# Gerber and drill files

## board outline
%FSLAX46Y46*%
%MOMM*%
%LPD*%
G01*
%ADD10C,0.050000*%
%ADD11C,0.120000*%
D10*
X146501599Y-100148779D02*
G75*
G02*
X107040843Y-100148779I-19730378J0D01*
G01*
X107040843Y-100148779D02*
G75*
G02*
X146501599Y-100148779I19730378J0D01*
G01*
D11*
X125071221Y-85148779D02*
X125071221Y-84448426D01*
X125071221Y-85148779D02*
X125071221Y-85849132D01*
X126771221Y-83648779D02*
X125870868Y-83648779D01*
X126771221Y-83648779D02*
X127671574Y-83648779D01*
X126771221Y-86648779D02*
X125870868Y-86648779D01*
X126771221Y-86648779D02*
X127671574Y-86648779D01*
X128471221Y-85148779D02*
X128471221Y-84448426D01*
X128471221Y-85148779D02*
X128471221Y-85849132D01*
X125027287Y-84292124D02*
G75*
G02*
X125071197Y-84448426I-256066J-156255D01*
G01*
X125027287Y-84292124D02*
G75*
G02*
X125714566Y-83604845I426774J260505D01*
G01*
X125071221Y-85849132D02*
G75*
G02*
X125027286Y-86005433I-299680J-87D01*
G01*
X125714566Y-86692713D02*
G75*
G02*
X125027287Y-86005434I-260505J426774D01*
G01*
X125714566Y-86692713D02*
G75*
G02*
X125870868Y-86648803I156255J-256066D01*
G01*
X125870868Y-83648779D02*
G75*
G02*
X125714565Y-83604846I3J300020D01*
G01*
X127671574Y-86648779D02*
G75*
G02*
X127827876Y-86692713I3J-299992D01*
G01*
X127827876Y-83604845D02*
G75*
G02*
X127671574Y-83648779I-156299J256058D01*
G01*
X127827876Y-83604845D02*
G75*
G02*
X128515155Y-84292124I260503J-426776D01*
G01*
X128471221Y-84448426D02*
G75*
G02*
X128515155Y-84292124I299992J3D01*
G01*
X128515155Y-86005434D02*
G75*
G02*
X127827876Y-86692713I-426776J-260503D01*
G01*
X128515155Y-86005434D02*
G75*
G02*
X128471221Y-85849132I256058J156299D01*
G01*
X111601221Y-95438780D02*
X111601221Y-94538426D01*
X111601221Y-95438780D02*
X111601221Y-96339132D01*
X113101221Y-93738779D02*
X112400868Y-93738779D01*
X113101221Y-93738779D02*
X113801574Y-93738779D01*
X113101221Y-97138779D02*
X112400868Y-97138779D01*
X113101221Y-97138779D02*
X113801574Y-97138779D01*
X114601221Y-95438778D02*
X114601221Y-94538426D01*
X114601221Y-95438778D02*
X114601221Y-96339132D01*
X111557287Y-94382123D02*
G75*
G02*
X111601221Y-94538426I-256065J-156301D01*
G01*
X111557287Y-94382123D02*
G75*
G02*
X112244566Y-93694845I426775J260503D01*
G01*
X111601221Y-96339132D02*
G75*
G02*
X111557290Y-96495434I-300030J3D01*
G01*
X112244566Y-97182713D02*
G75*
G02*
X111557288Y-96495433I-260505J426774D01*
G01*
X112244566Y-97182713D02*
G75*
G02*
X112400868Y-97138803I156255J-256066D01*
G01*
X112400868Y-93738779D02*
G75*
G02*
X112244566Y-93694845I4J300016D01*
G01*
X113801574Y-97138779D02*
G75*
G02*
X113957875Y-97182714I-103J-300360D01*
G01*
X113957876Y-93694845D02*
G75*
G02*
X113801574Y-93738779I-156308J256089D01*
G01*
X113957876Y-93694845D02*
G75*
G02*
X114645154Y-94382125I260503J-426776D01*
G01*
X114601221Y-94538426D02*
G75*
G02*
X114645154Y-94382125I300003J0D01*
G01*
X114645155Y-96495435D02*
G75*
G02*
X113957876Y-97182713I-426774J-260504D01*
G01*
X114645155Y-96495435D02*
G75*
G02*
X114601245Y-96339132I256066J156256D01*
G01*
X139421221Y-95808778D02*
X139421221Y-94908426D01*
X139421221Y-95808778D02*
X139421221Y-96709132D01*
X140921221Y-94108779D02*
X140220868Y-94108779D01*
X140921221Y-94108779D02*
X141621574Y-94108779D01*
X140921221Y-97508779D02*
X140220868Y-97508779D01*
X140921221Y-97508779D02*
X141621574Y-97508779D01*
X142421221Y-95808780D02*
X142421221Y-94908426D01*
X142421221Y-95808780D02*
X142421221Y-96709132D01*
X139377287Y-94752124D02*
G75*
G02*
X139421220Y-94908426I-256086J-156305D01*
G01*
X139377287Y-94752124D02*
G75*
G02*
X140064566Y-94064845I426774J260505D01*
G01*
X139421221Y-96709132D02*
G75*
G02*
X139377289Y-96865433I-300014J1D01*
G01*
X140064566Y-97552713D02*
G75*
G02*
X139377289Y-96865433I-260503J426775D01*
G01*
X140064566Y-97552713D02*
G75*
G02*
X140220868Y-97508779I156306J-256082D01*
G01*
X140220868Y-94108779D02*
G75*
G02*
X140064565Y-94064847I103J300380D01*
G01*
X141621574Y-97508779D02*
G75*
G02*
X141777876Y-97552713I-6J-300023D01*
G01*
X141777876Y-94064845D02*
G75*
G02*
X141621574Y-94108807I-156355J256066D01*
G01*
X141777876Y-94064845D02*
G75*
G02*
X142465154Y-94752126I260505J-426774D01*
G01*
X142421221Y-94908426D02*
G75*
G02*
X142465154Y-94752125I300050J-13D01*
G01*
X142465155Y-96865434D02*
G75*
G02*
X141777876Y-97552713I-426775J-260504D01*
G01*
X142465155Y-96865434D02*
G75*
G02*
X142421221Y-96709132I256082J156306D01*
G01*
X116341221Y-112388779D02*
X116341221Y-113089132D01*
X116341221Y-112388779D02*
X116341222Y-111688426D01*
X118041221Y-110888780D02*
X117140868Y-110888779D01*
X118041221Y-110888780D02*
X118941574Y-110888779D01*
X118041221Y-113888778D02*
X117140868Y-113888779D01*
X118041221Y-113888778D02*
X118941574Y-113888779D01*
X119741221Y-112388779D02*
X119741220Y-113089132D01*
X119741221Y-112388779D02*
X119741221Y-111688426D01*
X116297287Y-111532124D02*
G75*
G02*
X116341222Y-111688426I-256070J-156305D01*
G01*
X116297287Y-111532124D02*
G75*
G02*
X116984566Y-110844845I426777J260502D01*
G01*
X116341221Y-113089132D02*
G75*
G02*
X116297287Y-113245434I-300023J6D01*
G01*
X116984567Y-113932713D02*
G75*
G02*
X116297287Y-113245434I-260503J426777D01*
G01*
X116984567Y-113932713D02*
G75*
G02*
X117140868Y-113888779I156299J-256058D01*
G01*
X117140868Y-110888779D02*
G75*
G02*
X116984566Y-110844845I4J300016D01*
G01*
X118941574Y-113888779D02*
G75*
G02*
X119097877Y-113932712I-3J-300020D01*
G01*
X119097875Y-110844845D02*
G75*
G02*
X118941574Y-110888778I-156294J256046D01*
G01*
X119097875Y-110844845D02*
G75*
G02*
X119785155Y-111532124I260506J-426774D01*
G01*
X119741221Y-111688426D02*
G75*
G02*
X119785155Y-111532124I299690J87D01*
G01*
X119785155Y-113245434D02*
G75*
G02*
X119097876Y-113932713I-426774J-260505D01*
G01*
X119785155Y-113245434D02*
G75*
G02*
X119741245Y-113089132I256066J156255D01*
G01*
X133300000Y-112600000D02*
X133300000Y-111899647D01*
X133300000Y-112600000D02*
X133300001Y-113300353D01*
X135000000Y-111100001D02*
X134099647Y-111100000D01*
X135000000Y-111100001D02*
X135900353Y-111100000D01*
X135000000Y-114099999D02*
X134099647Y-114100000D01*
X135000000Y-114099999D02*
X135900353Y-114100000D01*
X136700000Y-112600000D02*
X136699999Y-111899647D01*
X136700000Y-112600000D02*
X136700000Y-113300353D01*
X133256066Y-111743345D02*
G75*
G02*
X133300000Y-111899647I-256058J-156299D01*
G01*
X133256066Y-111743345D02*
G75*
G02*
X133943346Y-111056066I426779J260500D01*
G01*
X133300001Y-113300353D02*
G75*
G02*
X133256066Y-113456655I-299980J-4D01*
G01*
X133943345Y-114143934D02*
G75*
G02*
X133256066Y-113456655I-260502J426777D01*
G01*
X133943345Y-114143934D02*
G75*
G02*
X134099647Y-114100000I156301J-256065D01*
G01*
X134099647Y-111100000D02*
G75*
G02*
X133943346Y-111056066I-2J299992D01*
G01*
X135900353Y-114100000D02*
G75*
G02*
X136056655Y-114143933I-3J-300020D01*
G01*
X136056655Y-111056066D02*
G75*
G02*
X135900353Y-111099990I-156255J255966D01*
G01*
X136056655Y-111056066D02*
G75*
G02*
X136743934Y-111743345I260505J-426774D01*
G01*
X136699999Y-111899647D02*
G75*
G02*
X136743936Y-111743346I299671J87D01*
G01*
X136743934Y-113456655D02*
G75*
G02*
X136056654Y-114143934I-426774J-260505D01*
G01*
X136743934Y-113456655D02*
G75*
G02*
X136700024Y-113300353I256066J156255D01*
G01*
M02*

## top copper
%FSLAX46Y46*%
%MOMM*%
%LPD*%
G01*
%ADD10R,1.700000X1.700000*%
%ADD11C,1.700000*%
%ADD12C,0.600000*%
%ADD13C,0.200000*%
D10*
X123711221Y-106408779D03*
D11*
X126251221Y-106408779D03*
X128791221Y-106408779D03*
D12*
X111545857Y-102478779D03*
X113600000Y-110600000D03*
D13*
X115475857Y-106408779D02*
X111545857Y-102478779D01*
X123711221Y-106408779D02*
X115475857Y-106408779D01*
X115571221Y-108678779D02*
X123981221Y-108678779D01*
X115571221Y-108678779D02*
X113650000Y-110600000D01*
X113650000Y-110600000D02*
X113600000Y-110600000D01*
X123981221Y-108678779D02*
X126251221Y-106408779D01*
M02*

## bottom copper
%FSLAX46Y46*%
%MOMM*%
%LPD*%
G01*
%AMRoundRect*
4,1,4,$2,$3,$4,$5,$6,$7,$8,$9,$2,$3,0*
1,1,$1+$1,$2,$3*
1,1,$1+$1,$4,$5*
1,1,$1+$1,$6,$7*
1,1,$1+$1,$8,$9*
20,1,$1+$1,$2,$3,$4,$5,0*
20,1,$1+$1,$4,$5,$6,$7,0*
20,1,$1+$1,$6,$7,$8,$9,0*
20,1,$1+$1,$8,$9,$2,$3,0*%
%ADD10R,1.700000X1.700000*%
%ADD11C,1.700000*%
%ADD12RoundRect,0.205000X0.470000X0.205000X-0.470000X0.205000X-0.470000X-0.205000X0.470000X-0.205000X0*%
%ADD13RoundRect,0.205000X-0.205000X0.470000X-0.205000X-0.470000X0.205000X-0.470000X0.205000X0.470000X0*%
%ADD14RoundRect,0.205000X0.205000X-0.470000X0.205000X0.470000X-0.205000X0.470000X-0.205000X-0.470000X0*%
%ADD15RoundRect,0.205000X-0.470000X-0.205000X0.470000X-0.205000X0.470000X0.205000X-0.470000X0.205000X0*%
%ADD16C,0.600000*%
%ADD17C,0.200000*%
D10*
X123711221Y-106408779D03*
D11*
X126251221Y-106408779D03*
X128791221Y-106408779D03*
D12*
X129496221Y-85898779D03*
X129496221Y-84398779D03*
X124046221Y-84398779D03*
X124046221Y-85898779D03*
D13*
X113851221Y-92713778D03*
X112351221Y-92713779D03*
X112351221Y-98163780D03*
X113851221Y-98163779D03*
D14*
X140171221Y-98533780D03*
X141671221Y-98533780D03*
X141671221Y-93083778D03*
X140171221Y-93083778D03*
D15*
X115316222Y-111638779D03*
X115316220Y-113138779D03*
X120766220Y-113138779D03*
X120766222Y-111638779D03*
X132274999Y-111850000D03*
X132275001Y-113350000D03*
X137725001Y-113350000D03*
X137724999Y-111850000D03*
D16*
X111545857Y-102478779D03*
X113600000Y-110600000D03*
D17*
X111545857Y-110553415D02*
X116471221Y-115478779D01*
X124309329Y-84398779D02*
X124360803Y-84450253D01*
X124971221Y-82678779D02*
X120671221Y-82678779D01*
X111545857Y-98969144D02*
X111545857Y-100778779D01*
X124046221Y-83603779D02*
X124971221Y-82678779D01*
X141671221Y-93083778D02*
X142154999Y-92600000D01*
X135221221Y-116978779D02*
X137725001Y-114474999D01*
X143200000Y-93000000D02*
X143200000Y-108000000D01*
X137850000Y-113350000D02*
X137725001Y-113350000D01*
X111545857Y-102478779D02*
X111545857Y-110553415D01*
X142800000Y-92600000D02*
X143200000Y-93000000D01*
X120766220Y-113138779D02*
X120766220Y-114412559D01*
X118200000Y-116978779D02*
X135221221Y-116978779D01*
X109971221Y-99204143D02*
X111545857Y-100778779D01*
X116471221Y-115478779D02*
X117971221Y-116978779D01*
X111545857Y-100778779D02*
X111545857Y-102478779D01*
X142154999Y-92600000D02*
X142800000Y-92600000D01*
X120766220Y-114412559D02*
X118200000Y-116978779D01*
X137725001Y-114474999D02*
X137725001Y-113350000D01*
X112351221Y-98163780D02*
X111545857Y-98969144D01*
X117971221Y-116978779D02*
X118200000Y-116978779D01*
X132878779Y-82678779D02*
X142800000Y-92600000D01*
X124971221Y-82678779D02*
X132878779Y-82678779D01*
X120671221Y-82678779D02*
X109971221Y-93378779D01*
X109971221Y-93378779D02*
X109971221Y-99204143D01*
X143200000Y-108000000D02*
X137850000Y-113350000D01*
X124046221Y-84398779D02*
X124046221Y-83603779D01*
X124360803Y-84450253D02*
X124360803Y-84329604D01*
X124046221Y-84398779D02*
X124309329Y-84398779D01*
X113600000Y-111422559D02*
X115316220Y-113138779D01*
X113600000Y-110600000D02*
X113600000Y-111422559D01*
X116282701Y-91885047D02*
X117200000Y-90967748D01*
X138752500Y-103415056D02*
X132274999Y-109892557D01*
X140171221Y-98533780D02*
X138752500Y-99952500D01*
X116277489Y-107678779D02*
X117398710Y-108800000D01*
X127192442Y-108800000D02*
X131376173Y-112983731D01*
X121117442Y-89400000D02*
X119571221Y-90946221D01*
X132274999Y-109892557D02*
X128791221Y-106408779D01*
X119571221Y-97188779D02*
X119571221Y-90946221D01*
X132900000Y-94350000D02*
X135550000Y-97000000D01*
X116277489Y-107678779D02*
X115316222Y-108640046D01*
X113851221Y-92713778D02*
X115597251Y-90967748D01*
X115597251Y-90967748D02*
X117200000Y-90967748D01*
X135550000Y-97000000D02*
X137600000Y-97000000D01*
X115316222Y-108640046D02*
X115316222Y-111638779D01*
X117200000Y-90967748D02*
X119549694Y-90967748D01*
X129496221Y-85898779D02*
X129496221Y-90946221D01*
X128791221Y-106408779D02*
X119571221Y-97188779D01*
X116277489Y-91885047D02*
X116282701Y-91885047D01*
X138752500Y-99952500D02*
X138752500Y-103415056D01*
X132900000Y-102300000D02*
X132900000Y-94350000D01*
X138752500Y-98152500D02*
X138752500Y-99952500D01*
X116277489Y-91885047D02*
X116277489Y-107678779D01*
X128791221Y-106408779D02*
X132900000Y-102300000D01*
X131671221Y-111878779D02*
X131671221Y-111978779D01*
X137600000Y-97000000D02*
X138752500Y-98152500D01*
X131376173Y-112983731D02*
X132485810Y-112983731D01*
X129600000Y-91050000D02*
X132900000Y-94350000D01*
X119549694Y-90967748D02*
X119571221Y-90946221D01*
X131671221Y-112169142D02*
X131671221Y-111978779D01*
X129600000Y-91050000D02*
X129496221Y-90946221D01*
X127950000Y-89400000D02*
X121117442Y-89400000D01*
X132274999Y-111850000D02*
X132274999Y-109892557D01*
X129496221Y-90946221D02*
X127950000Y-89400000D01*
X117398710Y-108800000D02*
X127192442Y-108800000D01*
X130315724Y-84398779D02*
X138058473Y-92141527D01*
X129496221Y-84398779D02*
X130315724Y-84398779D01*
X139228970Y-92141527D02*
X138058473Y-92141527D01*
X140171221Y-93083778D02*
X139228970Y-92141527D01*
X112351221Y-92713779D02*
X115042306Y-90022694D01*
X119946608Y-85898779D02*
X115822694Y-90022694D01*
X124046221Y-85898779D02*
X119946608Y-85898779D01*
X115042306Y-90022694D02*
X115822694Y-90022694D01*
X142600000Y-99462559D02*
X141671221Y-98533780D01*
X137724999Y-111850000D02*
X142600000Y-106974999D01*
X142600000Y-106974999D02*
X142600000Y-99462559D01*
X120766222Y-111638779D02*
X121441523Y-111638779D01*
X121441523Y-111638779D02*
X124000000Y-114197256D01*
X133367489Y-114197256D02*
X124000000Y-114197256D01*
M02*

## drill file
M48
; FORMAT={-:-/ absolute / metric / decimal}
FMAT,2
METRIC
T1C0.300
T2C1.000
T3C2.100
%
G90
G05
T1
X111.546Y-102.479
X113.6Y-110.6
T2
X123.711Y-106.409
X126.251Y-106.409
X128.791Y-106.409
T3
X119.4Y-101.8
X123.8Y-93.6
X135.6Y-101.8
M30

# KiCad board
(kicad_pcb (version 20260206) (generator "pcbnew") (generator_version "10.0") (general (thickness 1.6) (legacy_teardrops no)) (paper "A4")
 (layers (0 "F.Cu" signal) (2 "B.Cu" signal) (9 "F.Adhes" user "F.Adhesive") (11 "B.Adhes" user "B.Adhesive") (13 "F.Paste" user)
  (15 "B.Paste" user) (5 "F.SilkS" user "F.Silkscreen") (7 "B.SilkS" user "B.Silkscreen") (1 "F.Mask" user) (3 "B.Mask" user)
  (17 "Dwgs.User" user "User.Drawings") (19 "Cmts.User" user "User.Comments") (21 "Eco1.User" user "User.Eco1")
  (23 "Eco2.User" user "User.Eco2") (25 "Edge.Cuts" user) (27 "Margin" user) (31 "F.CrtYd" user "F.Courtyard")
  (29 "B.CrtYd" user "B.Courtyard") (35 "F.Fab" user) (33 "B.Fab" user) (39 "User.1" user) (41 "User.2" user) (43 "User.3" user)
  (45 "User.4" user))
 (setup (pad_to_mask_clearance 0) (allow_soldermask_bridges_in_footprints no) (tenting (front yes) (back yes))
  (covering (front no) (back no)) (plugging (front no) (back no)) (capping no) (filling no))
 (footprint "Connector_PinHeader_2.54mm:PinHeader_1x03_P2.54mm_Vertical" (layer "F.Cu") (at 123.711221 106.408779 90)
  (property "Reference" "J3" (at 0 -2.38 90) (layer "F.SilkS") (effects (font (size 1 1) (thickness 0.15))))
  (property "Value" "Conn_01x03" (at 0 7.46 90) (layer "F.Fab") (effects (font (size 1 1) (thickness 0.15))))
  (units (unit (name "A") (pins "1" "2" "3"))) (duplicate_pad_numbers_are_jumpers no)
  (pad "1" thru_hole rect (at 0 0 90) (size 1.7 1.7) (drill 1) (layers "*.Cu" "*.Mask") (remove_unused_layers no) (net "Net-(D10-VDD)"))
  (pad "2" thru_hole circle (at 0 2.54 90) (size 1.7 1.7) (drill 1) (layers "*.Cu" "*.Mask") (remove_unused_layers no) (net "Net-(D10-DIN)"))
  (pad "3" thru_hole circle (at 0 5.08 90) (size 1.7 1.7) (drill 1) (layers "*.Cu" "*.Mask") (remove_unused_layers no) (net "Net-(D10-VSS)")))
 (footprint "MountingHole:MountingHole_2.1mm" (layer "F.Cu") (at 135.6 101.8)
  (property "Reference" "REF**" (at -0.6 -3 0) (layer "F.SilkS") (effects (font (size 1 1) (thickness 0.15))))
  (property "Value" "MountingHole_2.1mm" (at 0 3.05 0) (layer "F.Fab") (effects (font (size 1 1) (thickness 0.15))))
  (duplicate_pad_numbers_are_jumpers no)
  (pad "" np_thru_hole circle (at 0 0) (size 2.1 2.1) (drill 2.1) (layers "*.Cu" "*.Mask")))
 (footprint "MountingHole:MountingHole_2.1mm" (layer "F.Cu") (at 123.8 93.6)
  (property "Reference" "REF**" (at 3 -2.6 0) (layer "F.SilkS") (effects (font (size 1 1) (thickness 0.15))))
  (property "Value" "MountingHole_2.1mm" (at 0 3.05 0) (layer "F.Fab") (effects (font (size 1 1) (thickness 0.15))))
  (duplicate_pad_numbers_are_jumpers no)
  (pad "" np_thru_hole circle (at 0 0) (size 2.1 2.1) (drill 2.1) (layers "*.Cu" "*.Mask")))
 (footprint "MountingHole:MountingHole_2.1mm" (layer "F.Cu") (at 119.4 101.8)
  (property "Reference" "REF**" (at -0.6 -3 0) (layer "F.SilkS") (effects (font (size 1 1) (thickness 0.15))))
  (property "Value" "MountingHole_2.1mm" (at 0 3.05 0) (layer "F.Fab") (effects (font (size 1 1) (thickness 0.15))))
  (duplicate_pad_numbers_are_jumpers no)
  (pad "" np_thru_hole circle (at 0 0) (size 2.1 2.1) (drill 2.1) (layers "*.Cu" "*.Mask")))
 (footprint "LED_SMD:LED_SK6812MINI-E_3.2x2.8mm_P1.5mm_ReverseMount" (layer "B.Cu") (at 126.771221 85.148779 180)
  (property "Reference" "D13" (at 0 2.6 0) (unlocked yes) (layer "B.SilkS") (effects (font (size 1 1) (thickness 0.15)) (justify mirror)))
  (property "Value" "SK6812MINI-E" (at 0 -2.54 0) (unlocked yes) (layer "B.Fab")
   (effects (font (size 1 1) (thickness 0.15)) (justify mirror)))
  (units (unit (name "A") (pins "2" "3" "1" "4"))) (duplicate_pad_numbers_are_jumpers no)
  (fp_line (start 1.7 0) (end 1.7 0.700353) (stroke (width 0.12) (type solid)) (layer "Edge.Cuts"))
  (fp_line (start 1.7 0) (end 1.7 -0.700353) (stroke (width 0.12) (type solid)) (layer "Edge.Cuts"))
  (fp_line (start 0 1.5) (end 0.900353 1.5) (stroke (width 0.12) (type solid)) (layer "Edge.Cuts"))
  (fp_line (start 0 1.5) (end -0.900353 1.5) (stroke (width 0.12) (type solid)) (layer "Edge.Cuts"))
  (fp_line (start 0 -1.5) (end 0.900353 -1.5) (stroke (width 0.12) (type solid)) (layer "Edge.Cuts"))
  (fp_line (start 0 -1.5) (end -0.900353 -1.5) (stroke (width 0.12) (type solid)) (layer "Edge.Cuts"))
  (fp_line (start -1.7 0) (end -1.7 0.700353) (stroke (width 0.12) (type solid)) (layer "Edge.Cuts"))
  (fp_line (start -1.7 0) (end -1.7 -0.700353) (stroke (width 0.12) (type solid)) (layer "Edge.Cuts"))
  (fp_arc (start 1.743934 0.856655) (mid 1.711191 0.781533) (end 1.7 0.700353) (stroke (width 0.12) (type solid)) (layer "Edge.Cuts"))
  (fp_arc (start 1.743934 0.856655) (mid 1.670713 1.470713) (end 1.056655 1.543934) (stroke (width 0.12) (type solid)) (layer "Edge.Cuts"))
  (fp_arc (start 1.7 -0.700353) (mid 1.711181 -0.781538) (end 1.743934 -0.856655) (stroke (width 0.12) (type solid)) (layer "Edge.Cuts"))
  (fp_arc (start 1.056655 -1.543934) (mid 1.670711 -1.470711) (end 1.743934 -0.856655) (stroke (width 0.12) (type solid))
   (layer "Edge.Cuts"))
  (fp_arc (start 1.056655 -1.543934) (mid 0.981533 -1.511191) (end 0.900353 -1.5) (stroke (width 0.12) (type solid)) (layer "Edge.Cuts"))
  (fp_arc (start 0.900353 1.5) (mid 0.981532 1.511193) (end 1.056655 1.543934) (stroke (width 0.12) (type solid)) (layer "Edge.Cuts"))
  (fp_arc (start -0.900353 -1.5) (mid -0.981533 -1.511192) (end -1.056655 -1.543934) (stroke (width 0.12) (type solid)) (layer "Edge.Cuts"))
  (fp_arc (start -1.056655 1.543934) (mid -0.981533 1.511192) (end -0.900353 1.5) (stroke (width 0.12) (type solid)) (layer "Edge.Cuts"))
  (fp_arc (start -1.056655 1.543934) (mid -1.670711 1.470711) (end -1.743934 0.856655) (stroke (width 0.12) (type solid))
   (layer "Edge.Cuts"))
  (fp_arc (start -1.7 0.700353) (mid -1.711192 0.781533) (end -1.743934 0.856655) (stroke (width 0.12) (type solid)) (layer "Edge.Cuts"))
  (fp_arc (start -1.743934 -0.856655) (mid -1.670711 -1.470711) (end -1.056655 -1.543934) (stroke (width 0.12) (type solid))
   (layer "Edge.Cuts"))
  (fp_arc (start -1.743934 -0.856655) (mid -1.711192 -0.781533) (end -1.7 -0.700353) (stroke (width 0.12) (type solid)) (layer "Edge.Cuts"))
  (pad "1" smd roundrect (at -2.725 -0.75 180) (size 1.35 0.82) (layers "B.Cu" "B.Mask" "B.Paste") (roundrect_rratio 0.25)
   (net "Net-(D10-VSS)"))
  (pad "2" smd roundrect (at -2.725 0.75 180) (size 1.35 0.82) (layers "B.Cu" "B.Mask" "B.Paste") (roundrect_rratio 0.25)
   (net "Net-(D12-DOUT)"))
  (pad "3" smd roundrect (at 2.725 0.75 180) (size 1.35 0.82) (layers "B.Cu" "B.Mask" "B.Paste") (roundrect_rratio 0.25)
   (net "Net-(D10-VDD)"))
  (pad "4" smd roundrect (at 2.725 -0.75 180) (size 1.35 0.82) (layers "B.Cu" "B.Mask" "B.Paste") (roundrect_rratio 0.25)
   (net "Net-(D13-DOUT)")))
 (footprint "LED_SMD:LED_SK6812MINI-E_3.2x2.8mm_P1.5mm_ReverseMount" (layer "B.Cu") (at 113.101221 95.438779 -90)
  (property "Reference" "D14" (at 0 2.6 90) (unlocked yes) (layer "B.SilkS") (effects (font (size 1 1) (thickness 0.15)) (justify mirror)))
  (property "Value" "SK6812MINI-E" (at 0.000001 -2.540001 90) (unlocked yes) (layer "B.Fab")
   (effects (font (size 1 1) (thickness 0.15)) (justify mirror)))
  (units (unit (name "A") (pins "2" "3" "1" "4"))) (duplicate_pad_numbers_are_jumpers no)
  (fp_line (start 0.000001 1.5) (end -0.900353 1.5) (stroke (width 0.12) (type solid)) (layer "Edge.Cuts"))
  (fp_line (start 0.000001 1.5) (end 0.900353 1.5) (stroke (width 0.12) (type solid)) (layer "Edge.Cuts"))
  (fp_line (start -1.7 0) (end -1.7 0.700353) (stroke (width 0.12) (type solid)) (layer "Edge.Cuts"))
  (fp_line (start -1.7 0) (end -1.7 -0.700353) (stroke (width 0.12) (type solid)) (layer "Edge.Cuts"))
  (fp_line (start 1.7 0) (end 1.7 0.700353) (stroke (width 0.12) (type solid)) (layer "Edge.Cuts"))
  (fp_line (start 1.7 0) (end 1.7 -0.700353) (stroke (width 0.12) (type solid)) (layer "Edge.Cuts"))
  (fp_line (start -0.000001 -1.5) (end -0.900353 -1.5) (stroke (width 0.12) (type solid)) (layer "Edge.Cuts"))
  (fp_line (start -0.000001 -1.5) (end 0.900353 -1.5) (stroke (width 0.12) (type solid)) (layer "Edge.Cuts"))
  (fp_arc (start -1.056656 1.543934) (mid -0.981533 1.511192) (end -0.900353 1.5) (stroke (width 0.12) (type solid)) (layer "Edge.Cuts"))
  (fp_arc (start -1.056656 1.543934) (mid -1.670712 1.470711) (end -1.743934 0.856655) (stroke (width 0.12) (type solid))
   (layer "Edge.Cuts"))
  (fp_arc (start 0.900353 1.5) (mid 0.981532 1.511193) (end 1.056654 1.543933) (stroke (width 0.12) (type solid)) (layer "Edge.Cuts"))
  (fp_arc (start 1.743934 0.856655) (mid 1.670712 1.470713) (end 1.056654 1.543933) (stroke (width 0.12) (type solid)) (layer "Edge.Cuts"))
  (fp_arc (start 1.743934 0.856655) (mid 1.711192 0.781533) (end 1.7 0.700353) (stroke (width 0.12) (type solid)) (layer "Edge.Cuts"))
  (fp_arc (start -1.7 0.700353) (mid -1.711193 0.781533) (end -1.743934 0.856655) (stroke (width 0.12) (type solid)) (layer "Edge.Cuts"))
  (fp_arc (start 1.7 -0.700353) (mid 1.711205 -0.781526) (end 1.743934 -0.856655) (stroke (width 0.12) (type solid)) (layer "Edge.Cuts"))
  (fp_arc (start -1.743934 -0.856655) (mid -1.711193 -0.781532) (end -1.7 -0.700353) (stroke (width 0.12) (type solid)) (layer "Edge.Cuts"))
  (fp_arc (start -1.743934 -0.856655) (mid -1.67071 -1.470712) (end -1.056654 -1.543933) (stroke (width 0.12) (type solid))
   (layer "Edge.Cuts"))
  (fp_arc (start -0.900353 -1.5) (mid -0.981532 -1.511192) (end -1.056654 -1.543933) (stroke (width 0.12) (type solid)) (layer "Edge.Cuts"))
  (fp_arc (start 1.056656 -1.543934) (mid 1.670712 -1.470711) (end 1.743934 -0.856655) (stroke (width 0.12) (type solid))
   (layer "Edge.Cuts"))
  (fp_arc (start 1.056656 -1.543934) (mid 0.981533 -1.511191) (end 0.900353 -1.5) (stroke (width 0.12) (type solid)) (layer "Edge.Cuts"))
  (pad "1" smd roundrect (at -2.725001 -0.75 270) (size 1.35 0.82) (layers "B.Cu" "B.Mask" "B.Paste") (roundrect_rratio 0.25)
   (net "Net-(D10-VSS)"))
  (pad "2" smd roundrect (at -2.725 0.75 270) (size 1.35 0.82) (layers "B.Cu" "B.Mask" "B.Paste") (roundrect_rratio 0.25)
   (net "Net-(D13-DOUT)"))
  (pad "3" smd roundrect (at 2.725001 0.75 270) (size 1.35 0.82) (layers "B.Cu" "B.Mask" "B.Paste") (roundrect_rratio 0.25)
   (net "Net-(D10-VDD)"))
  (pad "4" smd roundrect (at 2.725 -0.75 270) (size 1.35 0.82) (layers "B.Cu" "B.Mask" "B.Paste") (roundrect_rratio 0.25)
   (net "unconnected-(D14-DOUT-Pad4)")))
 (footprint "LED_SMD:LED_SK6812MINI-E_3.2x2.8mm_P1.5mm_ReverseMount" (layer "B.Cu") (at 140.921221 95.808779 90)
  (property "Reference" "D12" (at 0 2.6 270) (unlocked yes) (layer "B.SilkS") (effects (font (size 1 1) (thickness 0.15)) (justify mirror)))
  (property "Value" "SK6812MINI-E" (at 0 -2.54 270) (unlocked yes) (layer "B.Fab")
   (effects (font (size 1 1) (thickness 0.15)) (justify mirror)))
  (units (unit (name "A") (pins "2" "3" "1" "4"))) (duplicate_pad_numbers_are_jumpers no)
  (fp_line (start 0.000001 -1.5) (end 0.900353 -1.5) (stroke (width 0.12) (type solid)) (layer "Edge.Cuts"))
  (fp_line (start 0.000001 -1.5) (end -0.900353 -1.5) (stroke (width 0.12) (type solid)) (layer "Edge.Cuts"))
  (fp_line (start 1.7 0) (end 1.7 -0.700353) (stroke (width 0.12) (type solid)) (layer "Edge.Cuts"))
  (fp_line (start 1.7 0) (end 1.7 0.700353) (stroke (width 0.12) (type solid)) (layer "Edge.Cuts"))
  (fp_line (start -1.7 0) (end -1.7 -0.700353) (stroke (width 0.12) (type solid)) (layer "Edge.Cuts"))
  (fp_line (start -1.7 0) (end -1.7 0.700353) (stroke (width 0.12) (type solid)) (layer "Edge.Cuts"))
  (fp_line (start -0.000001 1.5) (end 0.900353 1.5) (stroke (width 0.12) (type solid)) (layer "Edge.Cuts"))
  (fp_line (start -0.000001 1.5) (end -0.900353 1.5) (stroke (width 0.12) (type solid)) (layer "Edge.Cuts"))
  (fp_arc (start 1.056655 -1.543934) (mid 0.981533 -1.511193) (end 0.900353 -1.5) (stroke (width 0.12) (type solid)) (layer "Edge.Cuts"))
  (fp_arc (start 1.056655 -1.543934) (mid 1.670711 -1.470712) (end 1.743934 -0.856655) (stroke (width 0.12) (type solid))
   (layer "Edge.Cuts"))
  (fp_arc (start -0.900353 -1.5) (mid -0.981532 -1.511192) (end -1.056654 -1.543932) (stroke (width 0.12) (type solid)) (layer "Edge.Cuts"))
  (fp_arc (start -1.743934 -0.856655) (mid -1.67071 -1.470712) (end -1.056654 -1.543932) (stroke (width 0.12) (type solid))
   (layer "Edge.Cuts"))
  (fp_arc (start -1.743934 -0.856655) (mid -1.711193 -0.781533) (end -1.7 -0.700353) (stroke (width 0.12) (type solid)) (layer "Edge.Cuts"))
  (fp_arc (start 1.7 -0.700353) (mid 1.711206 -0.781527) (end 1.743934 -0.856655) (stroke (width 0.12) (type solid)) (layer "Edge.Cuts"))
  (fp_arc (start -1.7 0.700353) (mid -1.711193 0.781532) (end -1.743934 0.856655) (stroke (width 0.12) (type solid)) (layer "Edge.Cuts"))
  (fp_arc (start 1.743934 0.856655) (mid 1.711193 0.781533) (end 1.7 0.700353) (stroke (width 0.12) (type solid)) (layer "Edge.Cuts"))
  (fp_arc (start 1.743934 0.856655) (mid 1.670712 1.470712) (end 1.056654 1.543932) (stroke (width 0.12) (type solid)) (layer "Edge.Cuts"))
  (fp_arc (start 0.900353 1.5) (mid 0.981531 1.511193) (end 1.056654 1.543932) (stroke (width 0.12) (type solid)) (layer "Edge.Cuts"))
  (fp_arc (start -1.056655 1.543934) (mid -1.670711 1.470712) (end -1.743934 0.856655) (stroke (width 0.12) (type solid))
   (layer "Edge.Cuts"))
  (fp_arc (start -1.056655 1.543934) (mid -0.981533 1.511193) (end -0.900353 1.5) (stroke (width 0.12) (type solid)) (layer "Edge.Cuts"))
  (pad "1" smd roundrect (at -2.725001 -0.75 90) (size 1.35 0.82) (layers "B.Cu" "B.Mask" "B.Paste") (roundrect_rratio 0.25)
   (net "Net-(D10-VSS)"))
  (pad "2" smd roundrect (at -2.725001 0.75 90) (size 1.35 0.82) (layers "B.Cu" "B.Mask" "B.Paste") (roundrect_rratio 0.25)
   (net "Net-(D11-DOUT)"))
  (pad "3" smd roundrect (at 2.725001 0.75 90) (size 1.35 0.82) (layers "B.Cu" "B.Mask" "B.Paste") (roundrect_rratio 0.25)
   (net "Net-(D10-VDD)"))
  (pad "4" smd roundrect (at 2.725001 -0.75 90) (size 1.35 0.82) (layers "B.Cu" "B.Mask" "B.Paste") (roundrect_rratio 0.25)
   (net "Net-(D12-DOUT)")))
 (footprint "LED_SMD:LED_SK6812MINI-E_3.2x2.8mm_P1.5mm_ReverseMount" (layer "B.Cu") (at 118.041221 112.388779)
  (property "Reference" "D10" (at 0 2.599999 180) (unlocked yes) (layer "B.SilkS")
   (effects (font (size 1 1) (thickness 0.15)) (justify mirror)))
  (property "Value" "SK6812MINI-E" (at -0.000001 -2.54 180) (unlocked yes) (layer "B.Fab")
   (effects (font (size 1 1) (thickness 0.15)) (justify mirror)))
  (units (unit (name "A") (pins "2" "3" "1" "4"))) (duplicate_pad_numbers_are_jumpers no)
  (fp_line (start -1.7 0) (end -1.7 0.700353) (stroke (width 0.12) (type solid)) (layer "Edge.Cuts"))
  (fp_line (start -1.7 0) (end -1.699999 -0.700353) (stroke (width 0.12) (type solid)) (layer "Edge.Cuts"))
  (fp_line (start 0 -1.499999) (end -0.900353 -1.5) (stroke (width 0.12) (type solid)) (layer "Edge.Cuts"))
  (fp_line (start 0 -1.499999) (end 0.900353 -1.5) (stroke (width 0.12) (type solid)) (layer "Edge.Cuts"))
  (fp_line (start 0 1.499999) (end -0.900353 1.5) (stroke (width 0.12) (type solid)) (layer "Edge.Cuts"))
  (fp_line (start 0 1.499999) (end 0.900353 1.5) (stroke (width 0.12) (type solid)) (layer "Edge.Cuts"))
  (fp_line (start 1.7 0) (end 1.699999 0.700353) (stroke (width 0.12) (type solid)) (layer "Edge.Cuts"))
  (fp_line (start 1.7 0) (end 1.7 -0.700353) (stroke (width 0.12) (type solid)) (layer "Edge.Cuts"))
  (fp_arc (start -1.743934 -0.856655) (mid -1.711192 -0.781533) (end -1.699999 -0.700353) (stroke (width 0.12) (type solid))
   (layer "Edge.Cuts"))
  (fp_arc (start -1.743934 -0.856655) (mid -1.67071 -1.470711) (end -1.056655 -1.543934) (stroke (width 0.12) (type solid))
   (layer "Edge.Cuts"))
  (fp_arc (start -1.7 0.700353) (mid -1.711193 0.781532) (end -1.743934 0.856655) (stroke (width 0.12) (type solid)) (layer "Edge.Cuts"))
  (fp_arc (start -1.056654 1.543934) (mid -1.67071 1.470711) (end -1.743934 0.856655) (stroke (width 0.12) (type solid)) (layer "Edge.Cuts"))
  (fp_arc (start -1.056654 1.543934) (mid -0.981532 1.511192) (end -0.900353 1.5) (stroke (width 0.12) (type solid)) (layer "Edge.Cuts"))
  (fp_arc (start -0.900353 -1.5) (mid -0.981533 -1.511193) (end -1.056655 -1.543934) (stroke (width 0.12) (type solid)) (layer "Edge.Cuts"))
  (fp_arc (start 0.900353 1.5) (mid 0.981532 1.511193) (end 1.056655 1.543934) (stroke (width 0.12) (type solid)) (layer "Edge.Cuts"))
  (fp_arc (start 1.056654 -1.543934) (mid 0.981533 -1.511192) (end 0.900353 -1.5) (stroke (width 0.12) (type solid)) (layer "Edge.Cuts"))
  (fp_arc (start 1.056654 -1.543934) (mid 1.67071 -1.470711) (end 1.743934 -0.856655) (stroke (width 0.12) (type solid)) (layer "Edge.Cuts"))
  (fp_arc (start 1.7 -0.700353) (mid 1.711181 -0.781537) (end 1.743934 -0.856655) (stroke (width 0.12) (type solid)) (layer "Edge.Cuts"))
  (fp_arc (start 1.743934 0.856655) (mid 1.670713 1.470713) (end 1.056655 1.543934) (stroke (width 0.12) (type solid)) (layer "Edge.Cuts"))
  (fp_arc (start 1.743934 0.856655) (mid 1.711191 0.781533) (end 1.699999 0.700353) (stroke (width 0.12) (type solid)) (layer "Edge.Cuts"))
  (pad "1" smd roundrect (at -2.724999 -0.75) (size 1.35 0.82) (layers "B.Cu" "B.Mask" "B.Paste") (roundrect_rratio 0.25)
   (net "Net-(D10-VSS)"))
  (pad "2" smd roundrect (at -2.725001 0.75) (size 1.35 0.82) (layers "B.Cu" "B.Mask" "B.Paste") (roundrect_rratio 0.25)
   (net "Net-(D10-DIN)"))
  (pad "3" smd roundrect (at 2.724999 0.75) (size 1.35 0.82) (layers "B.Cu" "B.Mask" "B.Paste") (roundrect_rratio 0.25)
   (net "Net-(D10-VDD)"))
  (pad "4" smd roundrect (at 2.725001 -0.75) (size 1.35 0.82) (layers "B.Cu" "B.Mask" "B.Paste") (roundrect_rratio 0.25)
   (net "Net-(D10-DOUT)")))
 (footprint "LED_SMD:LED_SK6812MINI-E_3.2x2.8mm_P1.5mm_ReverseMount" (layer "B.Cu") (at 135 112.6)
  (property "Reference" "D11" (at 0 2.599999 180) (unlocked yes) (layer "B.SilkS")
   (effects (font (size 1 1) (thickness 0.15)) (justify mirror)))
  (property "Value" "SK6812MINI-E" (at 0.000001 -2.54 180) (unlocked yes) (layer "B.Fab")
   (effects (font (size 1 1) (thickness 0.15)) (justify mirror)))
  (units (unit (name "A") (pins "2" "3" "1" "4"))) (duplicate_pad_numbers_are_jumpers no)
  (fp_line (start -1.7 0) (end -1.7 -0.700353) (stroke (width 0.12) (type solid)) (layer "Edge.Cuts"))
  (fp_line (start -1.7 0) (end -1.699999 0.700353) (stroke (width 0.12) (type solid)) (layer "Edge.Cuts"))
  (fp_line (start 0 -1.499999) (end -0.900353 -1.5) (stroke (width 0.12) (type solid)) (layer "Edge.Cuts"))
  (fp_line (start 0 -1.499999) (end 0.900353 -1.5) (stroke (width 0.12) (type solid)) (layer "Edge.Cuts"))
  (fp_line (start 0 1.499999) (end -0.900353 1.5) (stroke (width 0.12) (type solid)) (layer "Edge.Cuts"))
  (fp_line (start 0 1.499999) (end 0.900353 1.5) (stroke (width 0.12) (type solid)) (layer "Edge.Cuts"))
  (fp_line (start 1.7 0) (end 1.699999 -0.700353) (stroke (width 0.12) (type solid)) (layer "Edge.Cuts"))
  (fp_line (start 1.7 0) (end 1.7 0.700353) (stroke (width 0.12) (type solid)) (layer "Edge.Cuts"))
  (fp_arc (start -1.743934 -0.856655) (mid -1.711192 -0.781533) (end -1.7 -0.700353) (stroke (width 0.12) (type solid)) (layer "Edge.Cuts"))
  (fp_arc (start -1.743934 -0.856655) (mid -1.670709 -1.470709) (end -1.056654 -1.543934) (stroke (width 0.12) (type solid))
   (layer "Edge.Cuts"))
  (fp_arc (start -1.699999 0.700353) (mid -1.711191 0.781533) (end -1.743934 0.856655) (stroke (width 0.12) (type solid))
   (layer "Edge.Cuts"))
  (fp_arc (start -1.056655 1.543934) (mid -1.67071 1.470711) (end -1.743934 0.856655) (stroke (width 0.12) (type solid)) (layer "Edge.Cuts"))
  (fp_arc (start -1.056655 1.543934) (mid -0.981532 1.511192) (end -0.900353 1.5) (stroke (width 0.12) (type solid)) (layer "Edge.Cuts"))
  (fp_arc (start -0.900353 -1.5) (mid -0.981532 -1.511192) (end -1.056654 -1.543934) (stroke (width 0.12) (type solid)) (layer "Edge.Cuts"))
  (fp_arc (start 0.900353 1.5) (mid 0.981532 1.511193) (end 1.056654 1.543934) (stroke (width 0.12) (type solid)) (layer "Edge.Cuts"))
  (fp_arc (start 1.056655 -1.543934) (mid 0.981532 -1.51119) (end 0.900353 -1.5) (stroke (width 0.12) (type solid)) (layer "Edge.Cuts"))
  (fp_arc (start 1.056655 -1.543934) (mid 1.67071 -1.470711) (end 1.743934 -0.856655) (stroke (width 0.12) (type solid)) (layer "Edge.Cuts"))
  (fp_arc (start 1.699999 -0.700353) (mid 1.71118 -0.781538) (end 1.743934 -0.856655) (stroke (width 0.12) (type solid)) (layer "Edge.Cuts"))
  (fp_arc (start 1.743934 0.856655) (mid 1.670713 1.470712) (end 1.056654 1.543934) (stroke (width 0.12) (type solid)) (layer "Edge.Cuts"))
  (fp_arc (start 1.743934 0.856655) (mid 1.711191 0.781532) (end 1.7 0.700353) (stroke (width 0.12) (type solid)) (layer "Edge.Cuts"))
  (pad "1" smd roundrect (at -2.725001 -0.75) (size 1.35 0.82) (layers "B.Cu" "B.Mask" "B.Paste") (roundrect_rratio 0.25)
   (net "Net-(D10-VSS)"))
  (pad "2" smd roundrect (at -2.724999 0.75) (size 1.35 0.82) (layers "B.Cu" "B.Mask" "B.Paste") (roundrect_rratio 0.25)
   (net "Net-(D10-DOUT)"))
  (pad "3" smd roundrect (at 2.725001 0.75) (size 1.35 0.82) (layers "B.Cu" "B.Mask" "B.Paste") (roundrect_rratio 0.25)
   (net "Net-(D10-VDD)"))
  (pad "4" smd roundrect (at 2.724999 -0.75) (size 1.35 0.82) (layers "B.Cu" "B.Mask" "B.Paste") (roundrect_rratio 0.25)
   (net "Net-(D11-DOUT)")))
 (gr_circle (center 126.771221 100.148779) (end 146.5 100.4) (stroke (width 0.05) (type solid)) (fill no) (layer "Edge.Cuts"))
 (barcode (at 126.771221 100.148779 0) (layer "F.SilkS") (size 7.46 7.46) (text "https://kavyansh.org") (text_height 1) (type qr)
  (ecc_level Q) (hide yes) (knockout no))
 (segment (start 115.475857 106.408779) (end 111.545857 102.478779) (width 0.2) (layer "F.Cu") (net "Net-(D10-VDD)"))
 (segment (start 123.711221 106.408779) (end 115.475857 106.408779) (width 0.2) (layer "F.Cu") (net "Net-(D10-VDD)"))
 (via (at 111.545857 102.478779) (size 0.6) (drill 0.3) (layers "F.Cu" "B.Cu") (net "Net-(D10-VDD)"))
 (segment (start 111.545857 110.553415) (end 116.471221 115.478779) (width 0.2) (layer "B.Cu") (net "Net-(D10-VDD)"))
 (segment (start 124.309329 84.398779) (end 124.360803 84.450253) (width 0.2) (layer "B.Cu") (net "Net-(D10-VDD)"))
 (segment (start 124.971221 82.678779) (end 120.671221 82.678779) (width 0.2) (layer "B.Cu") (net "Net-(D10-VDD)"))
 (segment (start 111.545857 98.969144) (end 111.545857 100.778779) (width 0.2) (layer "B.Cu") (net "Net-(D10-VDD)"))
 (segment (start 124.046221 83.603779) (end 124.971221 82.678779) (width 0.2) (layer "B.Cu") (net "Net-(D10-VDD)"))
 (segment (start 141.671221 93.083778) (end 142.154999 92.6) (width 0.2) (layer "B.Cu") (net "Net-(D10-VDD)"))
 (segment (start 135.221221 116.978779) (end 137.725001 114.474999) (width 0.2) (layer "B.Cu") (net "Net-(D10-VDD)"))
 (segment (start 143.2 93) (end 143.2 108) (width 0.2) (layer "B.Cu") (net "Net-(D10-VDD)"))
 (segment (start 137.85 113.35) (end 137.725001 113.35) (width 0.2) (layer "B.Cu") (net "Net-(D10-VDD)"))
 (segment (start 111.545857 102.478779) (end 111.545857 110.553415) (width 0.2) (layer "B.Cu") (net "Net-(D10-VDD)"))
 (segment (start 142.8 92.6) (end 143.2 93) (width 0.2) (layer "B.Cu") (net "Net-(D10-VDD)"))
 (segment (start 120.76622 113.138779) (end 120.76622 114.412559) (width 0.2) (layer "B.Cu") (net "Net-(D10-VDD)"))
 (segment (start 118.2 116.978779) (end 135.221221 116.978779) (width 0.2) (layer "B.Cu") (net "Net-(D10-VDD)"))
 (segment (start 109.971221 99.204143) (end 111.545857 100.778779) (width 0.2) (layer "B.Cu") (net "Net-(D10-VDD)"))
 (segment (start 116.471221 115.478779) (end 117.971221 116.978779) (width 0.2) (layer "B.Cu") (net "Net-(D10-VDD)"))
 (segment (start 111.545857 100.778779) (end 111.545857 102.478779) (width 0.2) (layer "B.Cu") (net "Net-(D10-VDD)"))
 (segment (start 142.154999 92.6) (end 142.8 92.6) (width 0.2) (layer "B.Cu") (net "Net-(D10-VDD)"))
 (segment (start 120.76622 114.412559) (end 118.2 116.978779) (width 0.2) (layer "B.Cu") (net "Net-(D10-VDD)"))
 (segment (start 137.725001 114.474999) (end 137.725001 113.35) (width 0.2) (layer "B.Cu") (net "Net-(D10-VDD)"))
 (segment (start 112.351221 98.16378) (end 111.545857 98.969144) (width 0.2) (layer "B.Cu") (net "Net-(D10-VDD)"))
 (segment (start 117.971221 116.978779) (end 118.2 116.978779) (width 0.2) (layer "B.Cu") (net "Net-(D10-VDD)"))
 (segment (start 132.878779 82.678779) (end 142.8 92.6) (width 0.2) (layer "B.Cu") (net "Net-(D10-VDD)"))
 (segment (start 124.971221 82.678779) (end 132.878779 82.678779) (width 0.2) (layer "B.Cu") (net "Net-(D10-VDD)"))
 (segment (start 120.671221 82.678779) (end 109.971221 93.378779) (width 0.2) (layer "B.Cu") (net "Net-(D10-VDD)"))
 (segment (start 109.971221 93.378779) (end 109.971221 99.204143) (width 0.2) (layer "B.Cu") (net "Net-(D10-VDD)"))
 (segment (start 143.2 108) (end 137.85 113.35) (width 0.2) (layer "B.Cu") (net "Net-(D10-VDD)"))
 (segment (start 124.046221 84.398779) (end 124.046221 83.603779) (width 0.2) (layer "B.Cu") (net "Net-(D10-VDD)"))
 (segment (start 124.360803 84.450253) (end 124.360803 84.329604) (width 0.2) (layer "B.Cu") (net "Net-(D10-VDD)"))
 (segment (start 124.046221 84.398779) (end 124.309329 84.398779) (width 0.2) (layer "B.Cu") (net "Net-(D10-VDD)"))
 (segment (start 115.571221 108.678779) (end 123.981221 108.678779) (width 0.2) (layer "F.Cu") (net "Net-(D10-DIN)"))
 (segment (start 115.571221 108.678779) (end 113.65 110.6) (width 0.2) (layer "F.Cu") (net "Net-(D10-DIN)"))
 (segment (start 113.65 110.6) (end 113.6 110.6) (width 0.2) (layer "F.Cu") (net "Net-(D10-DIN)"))
 (segment (start 123.981221 108.678779) (end 126.251221 106.408779) (width 0.2) (layer "F.Cu") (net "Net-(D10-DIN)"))
 (via (at 113.6 110.6) (size 0.6) (drill 0.3) (layers "F.Cu" "B.Cu") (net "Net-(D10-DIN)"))
 (segment (start 113.6 111.422559) (end 115.31622 113.138779) (width 0.2) (layer "B.Cu") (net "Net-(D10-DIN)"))
 (segment (start 113.6 110.6) (end 113.6 111.422559) (width 0.2) (layer "B.Cu") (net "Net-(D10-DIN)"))
 (segment (start 116.282701 91.885047) (end 117.2 90.967748) (width 0.2) (layer "B.Cu") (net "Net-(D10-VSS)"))
 (segment (start 138.7525 103.415056) (end 132.274999 109.892557) (width 0.2) (layer "B.Cu") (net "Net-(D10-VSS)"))
 (segment (start 140.171221 98.53378) (end 138.7525 99.9525) (width 0.2) (layer "B.Cu") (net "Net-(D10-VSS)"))
 (segment (start 116.277489 107.678779) (end 117.39871 108.8) (width 0.2) (layer "B.Cu") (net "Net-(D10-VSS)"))
 (segment (start 127.192442 108.8) (end 131.376173 112.983731) (width 0.2) (layer "B.Cu") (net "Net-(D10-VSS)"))
 (segment (start 121.117442 89.4) (end 119.571221 90.946221) (width 0.2) (layer "B.Cu") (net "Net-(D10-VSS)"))
 (segment (start 132.274999 109.892557) (end 128.791221 106.408779) (width 0.2) (layer "B.Cu") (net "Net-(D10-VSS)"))
 (segment (start 119.571221 97.188779) (end 119.571221 90.946221) (width 0.2) (layer "B.Cu") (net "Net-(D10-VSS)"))
 (segment (start 132.9 94.35) (end 135.55 97) (width 0.2) (layer "B.Cu") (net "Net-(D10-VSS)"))
 (segment (start 116.277489 107.678779) (end 115.316222 108.640046) (width 0.2) (layer "B.Cu") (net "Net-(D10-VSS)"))
 (segment (start 113.851221 92.713778) (end 115.597251 90.967748) (width 0.2) (layer "B.Cu") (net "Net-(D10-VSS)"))
 (segment (start 115.597251 90.967748) (end 117.2 90.967748) (width 0.2) (layer "B.Cu") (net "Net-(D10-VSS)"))
 (segment (start 135.55 97) (end 137.6 97) (width 0.2) (layer "B.Cu") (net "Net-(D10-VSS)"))
 (segment (start 115.316222 108.640046) (end 115.316222 111.638779) (width 0.2) (layer "B.Cu") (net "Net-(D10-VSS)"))
 (segment (start 117.2 90.967748) (end 119.549694 90.967748) (width 0.2) (layer "B.Cu") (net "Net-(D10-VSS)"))
 (segment (start 129.496221 85.898779) (end 129.496221 90.946221) (width 0.2) (layer "B.Cu") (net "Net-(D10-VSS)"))
 (segment (start 128.791221 106.408779) (end 119.571221 97.188779) (width 0.2) (layer "B.Cu") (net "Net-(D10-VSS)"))
 (segment (start 116.277489 91.885047) (end 116.282701 91.885047) (width 0.2) (layer "B.Cu") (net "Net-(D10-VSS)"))
 (segment (start 138.7525 99.9525) (end 138.7525 103.415056) (width 0.2) (layer "B.Cu") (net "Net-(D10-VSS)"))
 (segment (start 132.9 102.3) (end 132.9 94.35) (width 0.2) (layer "B.Cu") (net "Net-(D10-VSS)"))
 (segment (start 138.7525 98.1525) (end 138.7525 99.9525) (width 0.2) (layer "B.Cu") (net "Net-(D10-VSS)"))
 (segment (start 116.277489 91.885047) (end 116.277489 107.678779) (width 0.2) (layer "B.Cu") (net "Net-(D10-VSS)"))
 (segment (start 128.791221 106.408779) (end 132.9 102.3) (width 0.2) (layer "B.Cu") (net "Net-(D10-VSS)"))
 (segment (start 131.671221 111.878779) (end 131.671221 111.978779) (width 0.2) (layer "B.Cu") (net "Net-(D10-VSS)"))
 (segment (start 137.6 97) (end 138.7525 98.1525) (width 0.2) (layer "B.Cu") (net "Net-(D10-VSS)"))
 (segment (start 131.376173 112.983731) (end 132.48581 112.983731) (width 0.2) (layer "B.Cu") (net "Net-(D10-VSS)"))
 (segment (start 129.6 91.05) (end 132.9 94.35) (width 0.2) (layer "B.Cu") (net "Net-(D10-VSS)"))
 (segment (start 119.549694 90.967748) (end 119.571221 90.946221) (width 0.2) (layer "B.Cu") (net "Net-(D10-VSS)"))
 (segment (start 131.671221 112.169142) (end 131.671221 111.978779) (width 0.2) (layer "B.Cu") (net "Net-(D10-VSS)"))
 (segment (start 129.6 91.05) (end 129.496221 90.946221) (width 0.2) (layer "B.Cu") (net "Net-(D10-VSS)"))
 (segment (start 127.95 89.4) (end 121.117442 89.4) (width 0.2) (layer "B.Cu") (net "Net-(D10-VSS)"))
 (segment (start 132.274999 111.85) (end 132.274999 109.892557) (width 0.2) (layer "B.Cu") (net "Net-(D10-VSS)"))
 (segment (start 129.496221 90.946221) (end 127.95 89.4) (width 0.2) (layer "B.Cu") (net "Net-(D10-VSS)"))
 (segment (start 117.39871 108.8) (end 127.192442 108.8) (width 0.2) (layer "B.Cu") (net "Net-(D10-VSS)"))
 (segment (start 130.315724 84.398779) (end 138.058473 92.141527) (width 0.2) (layer "B.Cu") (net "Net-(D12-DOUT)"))
 (segment (start 129.496221 84.398779) (end 130.315724 84.398779) (width 0.2) (layer "B.Cu") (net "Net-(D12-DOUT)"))
 (segment (start 139.22897 92.141527) (end 138.058473 92.141527) (width 0.2) (layer "B.Cu") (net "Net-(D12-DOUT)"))
 (segment (start 140.171221 93.083778) (end 139.22897 92.141527) (width 0.2) (layer "B.Cu") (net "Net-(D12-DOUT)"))
 (segment (start 112.351221 92.713779) (end 115.042306 90.022694) (width 0.2) (layer "B.Cu") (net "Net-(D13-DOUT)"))
 (segment (start 119.946608 85.898779) (end 115.822694 90.022694) (width 0.2) (layer "B.Cu") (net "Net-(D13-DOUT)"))
 (segment (start 124.046221 85.898779) (end 119.946608 85.898779) (width 0.2) (layer "B.Cu") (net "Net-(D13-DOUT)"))
 (segment (start 115.042306 90.022694) (end 115.822694 90.022694) (width 0.2) (layer "B.Cu") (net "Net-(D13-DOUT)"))
 (segment (start 142.6 99.462559) (end 141.671221 98.53378) (width 0.2) (layer "B.Cu") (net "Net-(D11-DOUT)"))
 (segment (start 137.724999 111.85) (end 142.6 106.974999) (width 0.2) (layer "B.Cu") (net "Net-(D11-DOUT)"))
 (segment (start 142.6 106.974999) (end 142.6 99.462559) (width 0.2) (layer "B.Cu") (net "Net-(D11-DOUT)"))
 (segment (start 120.766222 111.638779) (end 121.441523 111.638779) (width 0.2) (layer "B.Cu") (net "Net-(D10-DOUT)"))
 (segment (start 121.441523 111.638779) (end 124 114.197256) (width 0.2) (layer "B.Cu") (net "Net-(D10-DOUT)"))
 (segment (start 133.367489 114.197256) (end 124 114.197256) (width 0.2) (layer "B.Cu") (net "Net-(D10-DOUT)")))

